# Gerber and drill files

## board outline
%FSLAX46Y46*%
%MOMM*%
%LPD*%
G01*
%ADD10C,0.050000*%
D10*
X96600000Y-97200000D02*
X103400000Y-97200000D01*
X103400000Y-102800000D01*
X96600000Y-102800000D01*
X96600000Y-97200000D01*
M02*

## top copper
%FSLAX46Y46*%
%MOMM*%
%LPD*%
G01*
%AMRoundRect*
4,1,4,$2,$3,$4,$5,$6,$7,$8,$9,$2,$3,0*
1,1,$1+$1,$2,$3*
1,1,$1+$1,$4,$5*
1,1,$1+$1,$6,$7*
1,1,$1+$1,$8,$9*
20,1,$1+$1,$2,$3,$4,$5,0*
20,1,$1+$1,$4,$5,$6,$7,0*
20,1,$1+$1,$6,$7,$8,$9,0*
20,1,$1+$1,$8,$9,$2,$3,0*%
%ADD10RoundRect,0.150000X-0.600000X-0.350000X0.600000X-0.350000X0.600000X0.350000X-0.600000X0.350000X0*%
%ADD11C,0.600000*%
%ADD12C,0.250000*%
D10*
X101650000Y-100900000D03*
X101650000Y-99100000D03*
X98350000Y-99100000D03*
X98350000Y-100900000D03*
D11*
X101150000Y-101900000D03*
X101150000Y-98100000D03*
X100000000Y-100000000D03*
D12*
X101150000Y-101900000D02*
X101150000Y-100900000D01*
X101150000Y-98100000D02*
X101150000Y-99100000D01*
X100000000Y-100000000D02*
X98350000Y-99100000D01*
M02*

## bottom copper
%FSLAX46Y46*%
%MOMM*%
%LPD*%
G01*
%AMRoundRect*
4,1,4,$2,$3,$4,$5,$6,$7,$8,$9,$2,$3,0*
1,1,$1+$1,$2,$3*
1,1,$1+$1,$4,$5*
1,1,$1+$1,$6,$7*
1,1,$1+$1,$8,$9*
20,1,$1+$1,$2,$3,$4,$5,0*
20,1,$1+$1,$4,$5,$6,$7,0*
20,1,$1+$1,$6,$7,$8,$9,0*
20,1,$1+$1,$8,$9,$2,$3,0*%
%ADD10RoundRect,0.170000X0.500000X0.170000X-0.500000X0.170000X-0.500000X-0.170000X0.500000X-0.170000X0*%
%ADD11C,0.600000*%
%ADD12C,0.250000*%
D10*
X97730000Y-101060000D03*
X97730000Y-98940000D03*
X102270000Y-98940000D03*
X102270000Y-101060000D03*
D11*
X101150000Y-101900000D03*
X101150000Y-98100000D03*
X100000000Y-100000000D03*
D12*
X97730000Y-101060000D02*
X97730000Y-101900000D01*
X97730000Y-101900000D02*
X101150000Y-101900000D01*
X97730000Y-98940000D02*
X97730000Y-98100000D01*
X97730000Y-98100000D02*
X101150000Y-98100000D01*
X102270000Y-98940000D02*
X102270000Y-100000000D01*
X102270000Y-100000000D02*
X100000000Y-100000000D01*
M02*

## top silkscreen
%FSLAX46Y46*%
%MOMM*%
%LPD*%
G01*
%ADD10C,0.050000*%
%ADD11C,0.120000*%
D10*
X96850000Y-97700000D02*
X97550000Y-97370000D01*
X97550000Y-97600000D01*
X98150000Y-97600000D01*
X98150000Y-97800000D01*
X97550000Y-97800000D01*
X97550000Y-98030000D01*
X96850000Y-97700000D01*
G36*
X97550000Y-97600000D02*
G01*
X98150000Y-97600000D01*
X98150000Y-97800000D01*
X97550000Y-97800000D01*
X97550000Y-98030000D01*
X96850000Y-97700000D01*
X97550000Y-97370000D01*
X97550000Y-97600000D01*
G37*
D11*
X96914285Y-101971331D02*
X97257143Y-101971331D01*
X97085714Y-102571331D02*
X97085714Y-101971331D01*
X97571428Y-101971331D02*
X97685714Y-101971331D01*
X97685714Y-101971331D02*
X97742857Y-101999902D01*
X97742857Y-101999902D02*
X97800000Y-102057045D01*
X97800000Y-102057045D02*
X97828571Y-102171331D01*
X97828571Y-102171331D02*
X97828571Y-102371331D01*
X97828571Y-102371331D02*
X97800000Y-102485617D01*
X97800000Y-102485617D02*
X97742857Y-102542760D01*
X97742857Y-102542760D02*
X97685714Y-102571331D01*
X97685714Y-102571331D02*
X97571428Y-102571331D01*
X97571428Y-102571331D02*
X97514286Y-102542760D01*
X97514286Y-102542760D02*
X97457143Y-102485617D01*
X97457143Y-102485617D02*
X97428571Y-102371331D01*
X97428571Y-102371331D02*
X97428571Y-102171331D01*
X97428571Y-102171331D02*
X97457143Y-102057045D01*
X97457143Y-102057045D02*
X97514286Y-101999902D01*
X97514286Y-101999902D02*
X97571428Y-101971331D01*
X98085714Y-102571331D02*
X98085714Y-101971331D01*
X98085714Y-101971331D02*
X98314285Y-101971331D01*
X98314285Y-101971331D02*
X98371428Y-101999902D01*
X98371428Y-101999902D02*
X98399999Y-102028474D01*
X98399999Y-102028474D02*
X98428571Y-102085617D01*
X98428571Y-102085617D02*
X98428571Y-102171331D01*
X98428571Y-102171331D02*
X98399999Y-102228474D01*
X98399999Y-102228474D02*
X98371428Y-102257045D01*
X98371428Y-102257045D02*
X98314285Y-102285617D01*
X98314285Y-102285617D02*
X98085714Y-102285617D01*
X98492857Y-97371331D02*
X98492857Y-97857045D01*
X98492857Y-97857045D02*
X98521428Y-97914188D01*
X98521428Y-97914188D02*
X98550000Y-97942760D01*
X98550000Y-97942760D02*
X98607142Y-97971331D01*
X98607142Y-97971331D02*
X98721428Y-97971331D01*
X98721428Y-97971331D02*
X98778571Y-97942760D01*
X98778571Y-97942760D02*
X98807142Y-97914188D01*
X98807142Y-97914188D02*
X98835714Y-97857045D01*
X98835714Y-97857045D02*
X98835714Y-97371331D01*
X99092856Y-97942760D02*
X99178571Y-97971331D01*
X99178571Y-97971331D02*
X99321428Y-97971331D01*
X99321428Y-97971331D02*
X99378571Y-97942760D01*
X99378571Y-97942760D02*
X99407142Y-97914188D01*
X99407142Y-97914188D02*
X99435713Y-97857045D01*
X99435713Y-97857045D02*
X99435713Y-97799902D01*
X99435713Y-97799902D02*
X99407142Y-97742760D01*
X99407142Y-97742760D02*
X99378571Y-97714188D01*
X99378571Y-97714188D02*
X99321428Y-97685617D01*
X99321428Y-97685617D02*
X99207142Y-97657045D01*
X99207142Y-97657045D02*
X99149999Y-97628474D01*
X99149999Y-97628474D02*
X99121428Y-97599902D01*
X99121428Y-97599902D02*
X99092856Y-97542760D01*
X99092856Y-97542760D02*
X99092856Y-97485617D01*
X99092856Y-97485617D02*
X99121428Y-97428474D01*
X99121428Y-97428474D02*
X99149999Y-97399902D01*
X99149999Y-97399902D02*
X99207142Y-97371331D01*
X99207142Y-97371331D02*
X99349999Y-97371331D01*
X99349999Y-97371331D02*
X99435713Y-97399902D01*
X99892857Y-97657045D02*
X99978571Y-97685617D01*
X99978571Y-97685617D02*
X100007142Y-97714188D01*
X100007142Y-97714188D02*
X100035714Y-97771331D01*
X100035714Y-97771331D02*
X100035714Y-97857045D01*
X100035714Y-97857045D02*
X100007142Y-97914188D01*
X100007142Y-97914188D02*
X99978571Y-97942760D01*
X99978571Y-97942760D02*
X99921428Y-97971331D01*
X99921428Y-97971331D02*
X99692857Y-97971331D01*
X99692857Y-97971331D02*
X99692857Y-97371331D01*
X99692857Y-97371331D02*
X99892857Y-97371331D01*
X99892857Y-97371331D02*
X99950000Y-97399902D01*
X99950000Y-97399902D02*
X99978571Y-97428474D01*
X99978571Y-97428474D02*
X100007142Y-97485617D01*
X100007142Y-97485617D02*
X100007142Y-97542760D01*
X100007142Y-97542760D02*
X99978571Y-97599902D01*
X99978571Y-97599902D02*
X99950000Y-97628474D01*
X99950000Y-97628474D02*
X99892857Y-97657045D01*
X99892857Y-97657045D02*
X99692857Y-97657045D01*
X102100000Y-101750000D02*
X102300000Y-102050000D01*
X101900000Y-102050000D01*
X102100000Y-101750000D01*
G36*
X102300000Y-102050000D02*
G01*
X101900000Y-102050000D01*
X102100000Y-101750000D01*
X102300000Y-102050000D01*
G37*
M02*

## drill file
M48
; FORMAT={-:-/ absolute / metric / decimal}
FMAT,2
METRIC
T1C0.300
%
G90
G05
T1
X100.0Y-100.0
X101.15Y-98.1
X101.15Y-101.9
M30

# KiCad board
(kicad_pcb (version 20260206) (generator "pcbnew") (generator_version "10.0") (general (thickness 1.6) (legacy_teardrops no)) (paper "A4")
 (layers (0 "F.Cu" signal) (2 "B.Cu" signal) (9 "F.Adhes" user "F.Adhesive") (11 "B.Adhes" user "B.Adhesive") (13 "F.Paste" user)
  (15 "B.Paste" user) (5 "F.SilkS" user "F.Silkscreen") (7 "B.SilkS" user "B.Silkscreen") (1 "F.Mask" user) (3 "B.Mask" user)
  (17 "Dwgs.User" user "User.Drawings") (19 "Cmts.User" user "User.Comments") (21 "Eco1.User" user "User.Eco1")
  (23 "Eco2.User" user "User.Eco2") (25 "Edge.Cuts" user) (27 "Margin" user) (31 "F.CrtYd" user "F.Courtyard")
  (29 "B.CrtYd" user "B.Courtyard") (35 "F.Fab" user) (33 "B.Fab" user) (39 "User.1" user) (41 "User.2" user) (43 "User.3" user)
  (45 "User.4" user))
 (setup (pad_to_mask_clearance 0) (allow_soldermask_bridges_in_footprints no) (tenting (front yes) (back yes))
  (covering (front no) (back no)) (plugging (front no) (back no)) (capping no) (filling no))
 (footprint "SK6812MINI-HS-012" (layer "F.Cu") (at 100 100)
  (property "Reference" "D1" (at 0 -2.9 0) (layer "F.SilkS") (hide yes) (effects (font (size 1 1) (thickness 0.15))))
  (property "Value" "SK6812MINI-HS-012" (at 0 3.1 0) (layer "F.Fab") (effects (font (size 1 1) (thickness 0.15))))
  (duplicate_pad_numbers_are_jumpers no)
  (fp_poly (pts (xy 2.1 1.75) (xy 2.3 2.05) (xy 1.9 2.05)) (stroke (width 0.12) (type solid)) (fill yes) (layer "F.SilkS"))
  (pad "1" smd roundrect (at 1.65 0.9) (size 1.5 1) (layers "F.Cu" "F.Mask" "F.Paste") (roundrect_rratio 0.15) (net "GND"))
  (pad "2" smd roundrect (at 1.65 -0.9) (size 1.5 1) (layers "F.Cu" "F.Mask" "F.Paste") (roundrect_rratio 0.15) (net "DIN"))
  (pad "3" smd roundrect (at -1.65 -0.9) (size 1.5 1) (layers "F.Cu" "F.Mask" "F.Paste") (roundrect_rratio 0.15) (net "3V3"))
  (pad "4" smd roundrect (at -1.65 0.9) (size 1.5 1) (layers "F.Cu" "F.Mask" "F.Paste") (roundrect_rratio 0.15)))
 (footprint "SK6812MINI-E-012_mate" (layer "B.Cu") (at 100 100 180)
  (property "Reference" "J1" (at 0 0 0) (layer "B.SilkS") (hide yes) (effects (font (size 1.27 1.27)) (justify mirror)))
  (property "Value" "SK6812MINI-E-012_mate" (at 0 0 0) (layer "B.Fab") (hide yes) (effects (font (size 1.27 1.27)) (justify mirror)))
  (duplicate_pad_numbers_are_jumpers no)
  (pad "1" smd roundrect (at 2.27 -1.06 180) (size 1.34 0.68) (layers "B.Cu" "B.Mask" "B.Paste") (roundrect_rratio 0.25) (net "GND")
   (thermal_bridge_angle 45))
  (pad "2" smd roundrect (at 2.27 1.06 180) (size 1.34 0.68) (layers "B.Cu" "B.Mask" "B.Paste") (roundrect_rratio 0.25) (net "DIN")
   (thermal_bridge_angle 45))
  (pad "3" smd roundrect (at -2.27 1.06 180) (size 1.34 0.68) (layers "B.Cu" "B.Mask" "B.Paste") (roundrect_rratio 0.25) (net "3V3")
   (thermal_bridge_angle 45))
  (pad "4" smd roundrect (at -2.27 -1.06 180) (size 1.34 0.68) (layers "B.Cu" "B.Mask" "B.Paste") (roundrect_rratio 0.25)
   (thermal_bridge_angle 45)))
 (gr_poly
  (pts (xy 96.85 97.7) (xy 97.55 97.37) (xy 97.55 97.6) (xy 98.15 97.6) (xy 98.15 97.8) (xy 97.55 97.8) (xy 97.55 98.03))
  (stroke (width 0.05) (type default)) (fill yes) (layer "F.SilkS"))
 (gr_poly
  (pts (xy 96.6 97.2) (xy 103.4 97.2) (xy 103.4 102.8) (xy 96.6 102.8)) (stroke (width 0.05) (type default)) (fill no) (layer "Edge.Cuts"))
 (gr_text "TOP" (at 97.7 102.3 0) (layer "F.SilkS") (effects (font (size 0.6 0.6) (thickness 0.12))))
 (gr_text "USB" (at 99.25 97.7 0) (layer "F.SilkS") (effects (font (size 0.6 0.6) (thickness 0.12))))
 (segment (start 101.15 101.9) (end 101.15 100.9) (width 0.25) (layer "F.Cu") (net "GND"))
 (via (at 101.15 101.9) (size 0.6) (drill 0.3) (layers "F.Cu" "B.Cu") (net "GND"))
 (segment (start 97.73 101.06) (end 97.73 101.9) (width 0.25) (layer "B.Cu") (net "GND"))
 (segment (start 97.73 101.9) (end 101.15 101.9) (width 0.25) (layer "B.Cu") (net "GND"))
 (segment (start 101.15 98.1) (end 101.15 99.1) (width 0.25) (layer "F.Cu") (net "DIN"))
 (via (at 101.15 98.1) (size 0.6) (drill 0.3) (layers "F.Cu" "B.Cu") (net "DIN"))
 (segment (start 97.73 98.94) (end 97.73 98.1) (width 0.25) (layer "B.Cu") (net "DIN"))
 (segment (start 97.73 98.1) (end 101.15 98.1) (width 0.25) (layer "B.Cu") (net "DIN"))
 (segment (start 100 100) (end 98.35 99.1) (width 0.25) (layer "F.Cu") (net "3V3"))
 (via (at 100 100) (size 0.6) (drill 0.3) (layers "F.Cu" "B.Cu") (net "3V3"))
 (segment (start 102.27 98.94) (end 102.27 100) (width 0.25) (layer "B.Cu") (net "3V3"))
 (segment (start 102.27 100) (end 100 100) (width 0.25) (layer "B.Cu") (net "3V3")))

